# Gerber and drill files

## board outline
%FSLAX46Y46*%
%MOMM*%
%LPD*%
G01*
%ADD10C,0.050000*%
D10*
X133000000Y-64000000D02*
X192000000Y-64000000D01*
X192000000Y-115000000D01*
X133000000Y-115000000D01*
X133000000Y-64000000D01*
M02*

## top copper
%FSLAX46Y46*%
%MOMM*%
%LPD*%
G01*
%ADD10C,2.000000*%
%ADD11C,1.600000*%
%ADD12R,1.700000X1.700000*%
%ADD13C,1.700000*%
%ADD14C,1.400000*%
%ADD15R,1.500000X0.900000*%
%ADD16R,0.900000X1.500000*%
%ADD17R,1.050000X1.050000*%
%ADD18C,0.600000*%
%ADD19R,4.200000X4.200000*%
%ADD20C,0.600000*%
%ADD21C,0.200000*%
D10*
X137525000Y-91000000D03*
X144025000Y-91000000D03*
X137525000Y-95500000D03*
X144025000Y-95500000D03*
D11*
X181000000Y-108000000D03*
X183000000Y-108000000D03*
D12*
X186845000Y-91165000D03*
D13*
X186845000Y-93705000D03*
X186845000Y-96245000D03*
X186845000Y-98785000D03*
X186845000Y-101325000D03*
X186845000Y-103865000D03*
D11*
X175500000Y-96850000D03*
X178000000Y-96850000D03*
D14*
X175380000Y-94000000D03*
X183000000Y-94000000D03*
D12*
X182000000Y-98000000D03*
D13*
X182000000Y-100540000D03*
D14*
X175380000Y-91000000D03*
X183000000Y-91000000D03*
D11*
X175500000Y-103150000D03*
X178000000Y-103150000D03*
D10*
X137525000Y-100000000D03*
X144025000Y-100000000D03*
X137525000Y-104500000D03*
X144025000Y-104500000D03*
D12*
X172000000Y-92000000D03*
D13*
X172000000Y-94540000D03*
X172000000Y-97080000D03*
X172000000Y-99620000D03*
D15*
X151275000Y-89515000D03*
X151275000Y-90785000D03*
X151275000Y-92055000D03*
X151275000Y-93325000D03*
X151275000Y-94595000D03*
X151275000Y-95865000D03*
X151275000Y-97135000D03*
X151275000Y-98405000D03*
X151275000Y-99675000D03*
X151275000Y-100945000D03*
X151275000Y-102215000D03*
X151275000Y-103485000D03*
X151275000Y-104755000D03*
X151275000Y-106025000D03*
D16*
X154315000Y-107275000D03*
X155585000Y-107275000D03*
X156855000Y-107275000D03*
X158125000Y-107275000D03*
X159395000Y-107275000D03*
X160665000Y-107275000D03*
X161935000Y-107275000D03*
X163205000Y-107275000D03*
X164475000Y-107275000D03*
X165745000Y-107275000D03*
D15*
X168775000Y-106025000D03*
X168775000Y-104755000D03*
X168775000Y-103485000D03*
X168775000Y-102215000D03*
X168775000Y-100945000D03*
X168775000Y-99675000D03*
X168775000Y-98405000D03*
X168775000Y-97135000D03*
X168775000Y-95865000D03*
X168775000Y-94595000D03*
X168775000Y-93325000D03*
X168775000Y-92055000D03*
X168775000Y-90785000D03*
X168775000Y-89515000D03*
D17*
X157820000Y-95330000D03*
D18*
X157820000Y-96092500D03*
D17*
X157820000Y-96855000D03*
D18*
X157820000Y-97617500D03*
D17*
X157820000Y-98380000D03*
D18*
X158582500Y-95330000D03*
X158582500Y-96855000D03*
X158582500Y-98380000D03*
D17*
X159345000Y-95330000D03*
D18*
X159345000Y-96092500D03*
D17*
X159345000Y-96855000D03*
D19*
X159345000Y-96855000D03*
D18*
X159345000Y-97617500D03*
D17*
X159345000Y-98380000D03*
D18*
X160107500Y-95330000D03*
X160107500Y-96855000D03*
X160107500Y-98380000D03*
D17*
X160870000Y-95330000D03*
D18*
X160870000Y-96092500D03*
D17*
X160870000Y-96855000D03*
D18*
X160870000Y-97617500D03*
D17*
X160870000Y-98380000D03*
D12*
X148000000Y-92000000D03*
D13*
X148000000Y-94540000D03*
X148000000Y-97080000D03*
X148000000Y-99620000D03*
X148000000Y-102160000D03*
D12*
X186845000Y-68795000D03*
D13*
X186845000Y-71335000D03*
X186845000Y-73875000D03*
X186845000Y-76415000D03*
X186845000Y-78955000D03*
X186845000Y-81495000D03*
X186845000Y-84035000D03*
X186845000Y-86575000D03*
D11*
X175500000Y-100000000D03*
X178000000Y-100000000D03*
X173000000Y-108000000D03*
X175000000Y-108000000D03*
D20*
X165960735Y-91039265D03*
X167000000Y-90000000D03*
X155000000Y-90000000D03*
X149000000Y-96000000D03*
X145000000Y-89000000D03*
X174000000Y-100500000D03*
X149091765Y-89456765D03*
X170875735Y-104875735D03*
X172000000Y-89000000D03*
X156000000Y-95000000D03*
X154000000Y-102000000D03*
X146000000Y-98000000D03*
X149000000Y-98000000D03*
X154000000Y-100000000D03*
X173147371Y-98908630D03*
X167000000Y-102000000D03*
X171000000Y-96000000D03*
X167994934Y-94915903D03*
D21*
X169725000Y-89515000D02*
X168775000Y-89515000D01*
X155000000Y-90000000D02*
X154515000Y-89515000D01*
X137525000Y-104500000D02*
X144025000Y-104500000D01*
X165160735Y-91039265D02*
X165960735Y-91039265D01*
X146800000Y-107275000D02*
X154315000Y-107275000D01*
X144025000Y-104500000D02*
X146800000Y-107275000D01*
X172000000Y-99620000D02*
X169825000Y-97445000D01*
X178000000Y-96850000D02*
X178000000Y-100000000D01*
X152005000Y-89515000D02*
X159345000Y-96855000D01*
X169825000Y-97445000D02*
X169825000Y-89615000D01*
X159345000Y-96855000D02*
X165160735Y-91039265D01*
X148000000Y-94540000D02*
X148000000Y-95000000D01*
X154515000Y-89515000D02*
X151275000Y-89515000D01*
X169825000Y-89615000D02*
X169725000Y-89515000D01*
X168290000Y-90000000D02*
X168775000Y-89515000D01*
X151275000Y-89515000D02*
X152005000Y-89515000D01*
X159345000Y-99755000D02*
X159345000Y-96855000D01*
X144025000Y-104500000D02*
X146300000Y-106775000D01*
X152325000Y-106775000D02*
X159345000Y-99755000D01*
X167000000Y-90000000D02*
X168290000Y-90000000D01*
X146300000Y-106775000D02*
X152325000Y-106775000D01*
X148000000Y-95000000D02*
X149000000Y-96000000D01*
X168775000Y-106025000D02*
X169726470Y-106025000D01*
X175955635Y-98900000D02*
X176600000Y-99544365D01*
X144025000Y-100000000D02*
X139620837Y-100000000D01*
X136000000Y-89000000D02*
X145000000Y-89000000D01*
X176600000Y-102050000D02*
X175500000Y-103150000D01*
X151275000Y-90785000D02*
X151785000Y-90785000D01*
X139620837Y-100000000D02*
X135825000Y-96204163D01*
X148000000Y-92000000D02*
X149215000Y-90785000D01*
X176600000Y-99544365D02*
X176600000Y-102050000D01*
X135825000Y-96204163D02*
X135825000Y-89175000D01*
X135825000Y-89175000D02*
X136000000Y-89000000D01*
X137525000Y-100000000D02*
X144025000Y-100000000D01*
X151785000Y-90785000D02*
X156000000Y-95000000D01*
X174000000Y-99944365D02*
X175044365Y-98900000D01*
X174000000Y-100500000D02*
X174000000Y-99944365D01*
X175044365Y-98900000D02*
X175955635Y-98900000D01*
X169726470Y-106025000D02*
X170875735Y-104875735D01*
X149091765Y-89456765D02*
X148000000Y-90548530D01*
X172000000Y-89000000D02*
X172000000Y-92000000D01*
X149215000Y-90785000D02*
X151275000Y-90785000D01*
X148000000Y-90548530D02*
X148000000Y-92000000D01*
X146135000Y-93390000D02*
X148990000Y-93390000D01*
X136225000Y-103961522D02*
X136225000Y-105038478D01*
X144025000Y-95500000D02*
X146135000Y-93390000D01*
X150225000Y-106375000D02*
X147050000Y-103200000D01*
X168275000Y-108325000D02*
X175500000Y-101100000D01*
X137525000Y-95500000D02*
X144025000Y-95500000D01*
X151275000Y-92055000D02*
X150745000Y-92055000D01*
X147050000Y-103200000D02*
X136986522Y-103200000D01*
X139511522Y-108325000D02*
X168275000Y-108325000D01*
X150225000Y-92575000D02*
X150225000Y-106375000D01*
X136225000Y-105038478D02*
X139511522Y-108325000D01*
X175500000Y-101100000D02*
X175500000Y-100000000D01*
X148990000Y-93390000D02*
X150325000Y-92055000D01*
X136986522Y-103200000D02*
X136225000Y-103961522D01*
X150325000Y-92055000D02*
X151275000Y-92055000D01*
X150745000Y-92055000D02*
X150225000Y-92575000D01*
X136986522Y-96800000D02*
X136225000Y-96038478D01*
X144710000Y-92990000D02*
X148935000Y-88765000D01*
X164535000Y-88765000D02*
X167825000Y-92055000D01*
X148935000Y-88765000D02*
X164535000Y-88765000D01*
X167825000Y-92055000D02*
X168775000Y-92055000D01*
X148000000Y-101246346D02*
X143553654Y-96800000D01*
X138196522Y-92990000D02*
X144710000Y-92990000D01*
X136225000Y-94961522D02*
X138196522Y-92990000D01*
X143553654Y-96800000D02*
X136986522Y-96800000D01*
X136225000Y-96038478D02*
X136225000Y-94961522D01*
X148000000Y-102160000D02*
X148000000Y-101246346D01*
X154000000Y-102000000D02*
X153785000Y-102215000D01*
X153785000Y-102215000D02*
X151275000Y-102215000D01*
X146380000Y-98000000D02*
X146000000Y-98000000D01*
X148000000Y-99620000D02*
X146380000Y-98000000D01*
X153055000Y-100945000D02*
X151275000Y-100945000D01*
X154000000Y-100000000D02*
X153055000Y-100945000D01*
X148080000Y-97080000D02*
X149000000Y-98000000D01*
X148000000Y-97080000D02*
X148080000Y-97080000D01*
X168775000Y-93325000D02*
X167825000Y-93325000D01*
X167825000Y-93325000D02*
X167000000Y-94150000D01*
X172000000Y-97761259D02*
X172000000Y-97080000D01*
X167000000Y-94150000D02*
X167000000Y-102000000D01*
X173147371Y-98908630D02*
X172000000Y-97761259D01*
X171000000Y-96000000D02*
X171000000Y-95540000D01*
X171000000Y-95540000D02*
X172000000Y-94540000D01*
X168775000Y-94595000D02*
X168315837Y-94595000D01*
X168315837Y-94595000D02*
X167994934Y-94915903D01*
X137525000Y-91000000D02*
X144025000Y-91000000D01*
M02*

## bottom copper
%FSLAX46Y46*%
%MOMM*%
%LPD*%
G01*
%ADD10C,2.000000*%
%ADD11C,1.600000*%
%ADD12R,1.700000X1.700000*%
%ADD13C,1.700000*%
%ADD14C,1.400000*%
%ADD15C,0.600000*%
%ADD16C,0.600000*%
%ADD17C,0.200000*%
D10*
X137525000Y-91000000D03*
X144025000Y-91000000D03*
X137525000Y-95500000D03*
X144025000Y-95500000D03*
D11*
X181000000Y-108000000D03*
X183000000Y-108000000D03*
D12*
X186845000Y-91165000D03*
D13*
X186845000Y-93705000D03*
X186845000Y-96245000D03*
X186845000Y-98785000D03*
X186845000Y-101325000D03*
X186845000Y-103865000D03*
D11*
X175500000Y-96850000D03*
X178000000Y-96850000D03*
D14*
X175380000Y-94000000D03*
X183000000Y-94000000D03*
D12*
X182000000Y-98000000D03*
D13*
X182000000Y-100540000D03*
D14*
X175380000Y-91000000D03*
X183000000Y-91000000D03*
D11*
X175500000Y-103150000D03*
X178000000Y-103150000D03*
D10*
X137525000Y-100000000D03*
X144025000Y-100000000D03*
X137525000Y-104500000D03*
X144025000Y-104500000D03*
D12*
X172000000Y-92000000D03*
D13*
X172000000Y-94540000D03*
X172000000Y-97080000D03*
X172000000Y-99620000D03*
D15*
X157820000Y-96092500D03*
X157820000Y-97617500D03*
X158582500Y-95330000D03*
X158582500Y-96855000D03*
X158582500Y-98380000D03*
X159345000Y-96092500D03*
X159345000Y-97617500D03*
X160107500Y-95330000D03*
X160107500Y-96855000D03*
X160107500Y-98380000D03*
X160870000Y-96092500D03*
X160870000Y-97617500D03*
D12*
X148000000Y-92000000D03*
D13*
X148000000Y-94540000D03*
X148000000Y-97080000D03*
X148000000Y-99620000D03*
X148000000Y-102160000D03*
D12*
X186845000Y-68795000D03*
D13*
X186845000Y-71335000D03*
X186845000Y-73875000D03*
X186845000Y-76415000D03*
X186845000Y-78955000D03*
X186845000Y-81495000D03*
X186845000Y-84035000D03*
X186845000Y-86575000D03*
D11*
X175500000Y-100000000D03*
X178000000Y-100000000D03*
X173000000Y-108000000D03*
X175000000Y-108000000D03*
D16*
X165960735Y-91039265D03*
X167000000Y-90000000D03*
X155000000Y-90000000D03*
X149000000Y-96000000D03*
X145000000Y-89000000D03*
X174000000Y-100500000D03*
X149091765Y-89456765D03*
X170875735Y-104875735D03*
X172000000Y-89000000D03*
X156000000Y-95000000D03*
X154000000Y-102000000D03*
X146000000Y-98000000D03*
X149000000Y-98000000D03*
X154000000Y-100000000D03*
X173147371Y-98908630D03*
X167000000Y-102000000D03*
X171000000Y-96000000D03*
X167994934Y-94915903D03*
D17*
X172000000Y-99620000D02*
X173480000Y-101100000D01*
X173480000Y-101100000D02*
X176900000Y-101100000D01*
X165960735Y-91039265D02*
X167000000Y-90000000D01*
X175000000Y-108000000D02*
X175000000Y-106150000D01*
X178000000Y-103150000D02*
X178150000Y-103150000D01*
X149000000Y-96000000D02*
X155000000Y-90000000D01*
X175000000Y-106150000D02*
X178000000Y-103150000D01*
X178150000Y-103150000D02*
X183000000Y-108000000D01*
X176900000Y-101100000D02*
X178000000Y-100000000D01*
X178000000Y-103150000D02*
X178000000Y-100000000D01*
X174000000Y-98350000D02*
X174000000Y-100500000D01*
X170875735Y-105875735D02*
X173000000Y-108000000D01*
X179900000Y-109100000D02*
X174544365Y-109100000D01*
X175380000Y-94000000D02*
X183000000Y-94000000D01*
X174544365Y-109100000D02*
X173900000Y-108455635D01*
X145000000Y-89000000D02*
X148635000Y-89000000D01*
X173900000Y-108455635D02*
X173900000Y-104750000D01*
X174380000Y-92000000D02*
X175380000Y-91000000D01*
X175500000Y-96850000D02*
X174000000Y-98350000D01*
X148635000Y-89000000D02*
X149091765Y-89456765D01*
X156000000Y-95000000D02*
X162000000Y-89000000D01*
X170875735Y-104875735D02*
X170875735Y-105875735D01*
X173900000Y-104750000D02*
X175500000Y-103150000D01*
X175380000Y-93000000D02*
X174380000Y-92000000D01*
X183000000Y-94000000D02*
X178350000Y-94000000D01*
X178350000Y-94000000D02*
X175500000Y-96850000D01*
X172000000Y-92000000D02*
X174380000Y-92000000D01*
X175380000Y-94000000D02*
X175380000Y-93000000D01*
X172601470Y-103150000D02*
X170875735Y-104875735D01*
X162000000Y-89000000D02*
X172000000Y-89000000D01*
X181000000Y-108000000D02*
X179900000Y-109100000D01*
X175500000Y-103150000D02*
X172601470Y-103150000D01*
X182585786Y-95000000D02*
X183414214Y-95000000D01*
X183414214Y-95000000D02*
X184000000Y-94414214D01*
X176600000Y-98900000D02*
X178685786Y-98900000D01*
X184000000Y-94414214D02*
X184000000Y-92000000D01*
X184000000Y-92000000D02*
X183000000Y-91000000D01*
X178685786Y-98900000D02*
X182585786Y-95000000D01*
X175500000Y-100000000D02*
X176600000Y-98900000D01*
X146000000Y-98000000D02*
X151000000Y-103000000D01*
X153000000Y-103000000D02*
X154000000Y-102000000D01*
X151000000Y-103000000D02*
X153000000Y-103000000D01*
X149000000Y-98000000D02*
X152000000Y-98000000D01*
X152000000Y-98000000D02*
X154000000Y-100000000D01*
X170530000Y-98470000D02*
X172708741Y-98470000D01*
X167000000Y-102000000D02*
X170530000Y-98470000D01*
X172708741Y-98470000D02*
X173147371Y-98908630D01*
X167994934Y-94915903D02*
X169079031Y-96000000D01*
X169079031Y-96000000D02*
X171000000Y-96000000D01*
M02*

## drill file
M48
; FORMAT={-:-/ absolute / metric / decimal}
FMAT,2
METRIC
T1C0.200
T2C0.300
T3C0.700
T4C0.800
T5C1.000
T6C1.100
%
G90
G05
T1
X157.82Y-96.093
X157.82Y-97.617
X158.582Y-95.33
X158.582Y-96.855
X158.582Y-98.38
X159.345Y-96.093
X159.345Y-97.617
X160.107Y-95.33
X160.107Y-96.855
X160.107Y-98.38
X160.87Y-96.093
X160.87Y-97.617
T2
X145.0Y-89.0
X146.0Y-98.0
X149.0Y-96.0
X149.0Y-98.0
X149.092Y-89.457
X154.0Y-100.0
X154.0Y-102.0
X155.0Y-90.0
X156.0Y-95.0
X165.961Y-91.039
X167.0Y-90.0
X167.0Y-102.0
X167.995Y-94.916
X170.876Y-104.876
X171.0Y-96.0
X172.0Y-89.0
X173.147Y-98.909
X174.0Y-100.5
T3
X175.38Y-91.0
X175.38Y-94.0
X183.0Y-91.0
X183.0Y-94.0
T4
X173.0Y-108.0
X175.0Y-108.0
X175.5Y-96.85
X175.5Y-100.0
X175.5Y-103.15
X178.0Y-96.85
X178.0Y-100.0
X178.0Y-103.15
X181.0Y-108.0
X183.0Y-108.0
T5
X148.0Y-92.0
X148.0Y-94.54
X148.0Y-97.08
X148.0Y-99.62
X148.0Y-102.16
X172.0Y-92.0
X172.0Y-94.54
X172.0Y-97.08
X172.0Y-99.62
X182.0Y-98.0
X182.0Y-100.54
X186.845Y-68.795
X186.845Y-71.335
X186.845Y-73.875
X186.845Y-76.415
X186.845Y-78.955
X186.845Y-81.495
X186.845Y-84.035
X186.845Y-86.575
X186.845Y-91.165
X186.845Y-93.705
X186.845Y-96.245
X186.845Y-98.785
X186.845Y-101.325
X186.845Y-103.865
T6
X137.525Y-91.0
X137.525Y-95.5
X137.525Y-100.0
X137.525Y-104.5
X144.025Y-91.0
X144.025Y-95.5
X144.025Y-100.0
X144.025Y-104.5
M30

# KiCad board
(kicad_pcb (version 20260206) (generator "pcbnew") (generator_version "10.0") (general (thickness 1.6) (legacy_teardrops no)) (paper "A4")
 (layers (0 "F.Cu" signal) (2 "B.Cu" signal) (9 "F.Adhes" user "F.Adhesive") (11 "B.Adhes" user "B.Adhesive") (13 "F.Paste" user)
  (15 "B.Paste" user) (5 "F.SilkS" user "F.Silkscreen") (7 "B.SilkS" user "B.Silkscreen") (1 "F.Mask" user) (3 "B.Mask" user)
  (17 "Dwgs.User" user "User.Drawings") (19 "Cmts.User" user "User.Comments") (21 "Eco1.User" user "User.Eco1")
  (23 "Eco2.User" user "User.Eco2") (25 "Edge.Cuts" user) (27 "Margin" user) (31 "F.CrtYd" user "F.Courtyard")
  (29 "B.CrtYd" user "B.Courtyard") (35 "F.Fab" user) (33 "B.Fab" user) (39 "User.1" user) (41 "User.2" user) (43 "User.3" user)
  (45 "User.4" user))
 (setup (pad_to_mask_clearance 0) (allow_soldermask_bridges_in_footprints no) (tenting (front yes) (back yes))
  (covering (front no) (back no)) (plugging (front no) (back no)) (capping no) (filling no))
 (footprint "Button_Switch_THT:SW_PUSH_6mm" (layer "F.Cu") (at 137.525 91)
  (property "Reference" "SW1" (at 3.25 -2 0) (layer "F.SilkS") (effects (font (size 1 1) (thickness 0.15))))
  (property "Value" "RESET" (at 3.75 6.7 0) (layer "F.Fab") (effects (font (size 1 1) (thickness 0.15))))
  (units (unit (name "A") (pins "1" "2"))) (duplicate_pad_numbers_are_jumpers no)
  (pad "1" thru_hole circle (at 0 0 90) (size 2 2) (drill 1.1) (layers "*.Cu" "*.Mask") (remove_unused_layers no)
   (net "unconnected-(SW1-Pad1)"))
  (pad "1" thru_hole circle (at 6.5 0 90) (size 2 2) (drill 1.1) (layers "*.Cu" "*.Mask") (remove_unused_layers no)
   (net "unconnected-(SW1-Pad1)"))
  (pad "2" thru_hole circle (at 0 4.5 90) (size 2 2) (drill 1.1) (layers "*.Cu" "*.Mask") (remove_unused_layers no) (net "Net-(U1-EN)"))
  (pad "2" thru_hole circle (at 6.5 4.5 90) (size 2 2) (drill 1.1) (layers "*.Cu" "*.Mask") (remove_unused_layers no) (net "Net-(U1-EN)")))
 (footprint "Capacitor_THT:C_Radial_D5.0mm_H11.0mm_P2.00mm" (layer "F.Cu") (at 181 108)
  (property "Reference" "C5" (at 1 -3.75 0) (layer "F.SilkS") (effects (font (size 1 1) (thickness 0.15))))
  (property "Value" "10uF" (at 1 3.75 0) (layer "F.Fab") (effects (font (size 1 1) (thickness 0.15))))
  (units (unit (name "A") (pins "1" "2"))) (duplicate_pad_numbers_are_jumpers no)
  (pad "1" thru_hole circle (at 0 0) (size 1.6 1.6) (drill 0.8) (layers "*.Cu" "*.Mask") (remove_unused_layers no) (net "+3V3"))
  (pad "2" thru_hole circle (at 2 0) (size 1.6 1.6) (drill 0.8) (layers "*.Cu" "*.Mask") (remove_unused_layers no) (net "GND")))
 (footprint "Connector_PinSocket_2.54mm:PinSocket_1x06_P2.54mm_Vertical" (layer "F.Cu") (at 186.845 91.165)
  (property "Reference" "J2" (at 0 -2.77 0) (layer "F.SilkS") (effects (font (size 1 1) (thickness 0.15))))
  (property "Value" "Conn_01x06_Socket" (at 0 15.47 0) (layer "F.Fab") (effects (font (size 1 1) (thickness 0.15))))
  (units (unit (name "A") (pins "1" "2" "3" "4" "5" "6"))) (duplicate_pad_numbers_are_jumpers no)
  (pad "1" thru_hole rect (at 0 0) (size 1.7 1.7) (drill 1) (layers "*.Cu" "*.Mask") (remove_unused_layers no)
   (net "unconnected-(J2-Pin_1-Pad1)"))
  (pad "2" thru_hole circle (at 0 2.54) (size 1.7 1.7) (drill 1) (layers "*.Cu" "*.Mask") (remove_unused_layers no)
   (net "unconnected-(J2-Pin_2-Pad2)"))
  (pad "3" thru_hole circle (at 0 5.08) (size 1.7 1.7) (drill 1) (layers "*.Cu" "*.Mask") (remove_unused_layers no)
   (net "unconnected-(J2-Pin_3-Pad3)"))
  (pad "4" thru_hole circle (at 0 7.62) (size 1.7 1.7) (drill 1) (layers "*.Cu" "*.Mask") (remove_unused_layers no)
   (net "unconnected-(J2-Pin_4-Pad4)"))
  (pad "5" thru_hole circle (at 0 10.16) (size 1.7 1.7) (drill 1) (layers "*.Cu" "*.Mask") (remove_unused_layers no)
   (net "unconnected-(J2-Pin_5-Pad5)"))
  (pad "6" thru_hole circle (at 0 12.7) (size 1.7 1.7) (drill 1) (layers "*.Cu" "*.Mask") (remove_unused_layers no)
   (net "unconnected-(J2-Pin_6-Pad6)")))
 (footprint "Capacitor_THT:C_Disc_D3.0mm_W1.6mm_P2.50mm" (layer "F.Cu") (at 175.5 96.85)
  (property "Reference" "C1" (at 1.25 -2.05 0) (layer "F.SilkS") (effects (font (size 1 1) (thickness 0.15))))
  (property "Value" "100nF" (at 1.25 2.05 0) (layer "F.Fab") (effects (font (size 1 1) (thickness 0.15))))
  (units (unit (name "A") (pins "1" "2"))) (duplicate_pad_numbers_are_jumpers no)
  (pad "1" thru_hole circle (at 0 0) (size 1.6 1.6) (drill 0.8) (layers "*.Cu" "*.Mask") (remove_unused_layers no) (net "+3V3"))
  (pad "2" thru_hole circle (at 2.5 0) (size 1.6 1.6) (drill 0.8) (layers "*.Cu" "*.Mask") (remove_unused_layers no) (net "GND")))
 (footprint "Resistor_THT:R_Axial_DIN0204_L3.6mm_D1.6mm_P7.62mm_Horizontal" (layer "F.Cu") (at 175.38 94)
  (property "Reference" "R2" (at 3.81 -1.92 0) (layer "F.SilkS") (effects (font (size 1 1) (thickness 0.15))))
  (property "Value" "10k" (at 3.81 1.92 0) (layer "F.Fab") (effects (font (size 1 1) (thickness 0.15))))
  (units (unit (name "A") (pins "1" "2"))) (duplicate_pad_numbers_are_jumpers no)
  (pad "1" thru_hole circle (at 0 0) (size 1.4 1.4) (drill 0.7) (layers "*.Cu" "*.Mask") (remove_unused_layers no) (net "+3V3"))
  (pad "2" thru_hole circle (at 7.62 0) (size 1.4 1.4) (drill 0.7) (layers "*.Cu" "*.Mask") (remove_unused_layers no) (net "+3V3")))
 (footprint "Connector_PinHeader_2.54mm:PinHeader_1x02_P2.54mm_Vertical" (layer "F.Cu") (at 182 98)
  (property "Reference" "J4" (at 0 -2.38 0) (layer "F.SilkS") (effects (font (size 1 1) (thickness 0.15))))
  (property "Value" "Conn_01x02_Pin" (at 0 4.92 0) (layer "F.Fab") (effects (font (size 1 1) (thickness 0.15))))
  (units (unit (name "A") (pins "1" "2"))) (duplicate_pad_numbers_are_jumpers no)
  (pad "1" thru_hole rect (at 0 0) (size 1.7 1.7) (drill 1) (layers "*.Cu" "*.Mask") (remove_unused_layers no) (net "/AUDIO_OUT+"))
  (pad "2" thru_hole circle (at 0 2.54) (size 1.7 1.7) (drill 1) (layers "*.Cu" "*.Mask") (remove_unused_layers no) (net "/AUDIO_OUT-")))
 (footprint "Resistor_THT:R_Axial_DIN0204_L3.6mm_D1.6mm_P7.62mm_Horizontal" (layer "F.Cu") (at 175.38 91)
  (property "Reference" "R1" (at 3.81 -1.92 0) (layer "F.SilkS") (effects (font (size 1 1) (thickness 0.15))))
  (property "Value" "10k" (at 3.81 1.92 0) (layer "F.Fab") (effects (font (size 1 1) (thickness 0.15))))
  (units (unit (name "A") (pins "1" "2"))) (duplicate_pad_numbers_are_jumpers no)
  (pad "1" thru_hole circle (at 0 0) (size 1.4 1.4) (drill 0.7) (layers "*.Cu" "*.Mask") (remove_unused_layers no) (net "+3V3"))
  (pad "2" thru_hole circle (at 7.62 0) (size 1.4 1.4) (drill 0.7) (layers "*.Cu" "*.Mask") (remove_unused_layers no) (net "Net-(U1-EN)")))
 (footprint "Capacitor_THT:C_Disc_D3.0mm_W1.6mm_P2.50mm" (layer "F.Cu") (at 175.5 103.15)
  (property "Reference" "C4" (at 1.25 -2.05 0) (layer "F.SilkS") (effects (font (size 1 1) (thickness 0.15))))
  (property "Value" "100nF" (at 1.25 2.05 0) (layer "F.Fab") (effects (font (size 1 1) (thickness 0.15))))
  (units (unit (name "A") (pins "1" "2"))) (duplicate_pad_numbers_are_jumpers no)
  (pad "1" thru_hole circle (at 0 0) (size 1.6 1.6) (drill 0.8) (layers "*.Cu" "*.Mask") (remove_unused_layers no) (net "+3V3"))
  (pad "2" thru_hole circle (at 2.5 0) (size 1.6 1.6) (drill 0.8) (layers "*.Cu" "*.Mask") (remove_unused_layers no) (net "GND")))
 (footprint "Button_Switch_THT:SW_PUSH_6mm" (layer "F.Cu") (at 137.525 100)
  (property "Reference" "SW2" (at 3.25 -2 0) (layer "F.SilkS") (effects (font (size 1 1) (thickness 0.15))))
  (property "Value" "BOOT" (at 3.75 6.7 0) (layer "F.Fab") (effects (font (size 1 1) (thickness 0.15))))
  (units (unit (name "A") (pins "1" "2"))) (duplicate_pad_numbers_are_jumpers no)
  (pad "1" thru_hole circle (at 0 0 90) (size 2 2) (drill 1.1) (layers "*.Cu" "*.Mask") (remove_unused_layers no) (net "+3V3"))
  (pad "1" thru_hole circle (at 6.5 0 90) (size 2 2) (drill 1.1) (layers "*.Cu" "*.Mask") (remove_unused_layers no) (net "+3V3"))
  (pad "2" thru_hole circle (at 0 4.5 90) (size 2 2) (drill 1.1) (layers "*.Cu" "*.Mask") (remove_unused_layers no) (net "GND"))
  (pad "2" thru_hole circle (at 6.5 4.5 90) (size 2 2) (drill 1.1) (layers "*.Cu" "*.Mask") (remove_unused_layers no) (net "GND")))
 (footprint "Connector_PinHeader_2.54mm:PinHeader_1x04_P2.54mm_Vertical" (layer "F.Cu") (at 172 92)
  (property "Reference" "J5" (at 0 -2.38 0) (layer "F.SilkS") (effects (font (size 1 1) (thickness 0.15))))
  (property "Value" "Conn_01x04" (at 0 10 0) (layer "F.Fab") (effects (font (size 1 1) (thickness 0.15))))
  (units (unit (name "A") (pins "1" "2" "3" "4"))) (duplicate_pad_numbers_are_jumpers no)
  (pad "1" thru_hole rect (at 0 0) (size 1.7 1.7) (drill 1) (layers "*.Cu" "*.Mask") (remove_unused_layers no) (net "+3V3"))
  (pad "2" thru_hole circle (at 0 2.54) (size 1.7 1.7) (drill 1) (layers "*.Cu" "*.Mask") (remove_unused_layers no) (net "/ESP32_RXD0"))
  (pad "3" thru_hole circle (at 0 5.08) (size 1.7 1.7) (drill 1) (layers "*.Cu" "*.Mask") (remove_unused_layers no) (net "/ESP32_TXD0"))
  (pad "4" thru_hole circle (at 0 7.62) (size 1.7 1.7) (drill 1) (layers "*.Cu" "*.Mask") (remove_unused_layers no) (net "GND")))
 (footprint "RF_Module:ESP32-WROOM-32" (layer "F.Cu") (at 160.025 97.765)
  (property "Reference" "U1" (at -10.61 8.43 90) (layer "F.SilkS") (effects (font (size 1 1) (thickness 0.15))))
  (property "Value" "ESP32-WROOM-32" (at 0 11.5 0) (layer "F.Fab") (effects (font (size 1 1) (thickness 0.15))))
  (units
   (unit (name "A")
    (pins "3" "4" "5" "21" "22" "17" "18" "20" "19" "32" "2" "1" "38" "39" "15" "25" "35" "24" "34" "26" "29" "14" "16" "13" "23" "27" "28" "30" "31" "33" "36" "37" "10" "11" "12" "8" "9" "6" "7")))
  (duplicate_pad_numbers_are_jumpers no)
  (pad "1" smd rect (at -8.75 -8.25) (size 1.5 0.9) (layers "F.Cu" "F.Mask" "F.Paste") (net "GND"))
  (pad "2" smd rect (at -8.75 -6.98) (size 1.5 0.9) (layers "F.Cu" "F.Mask" "F.Paste") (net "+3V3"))
  (pad "3" smd rect (at -8.75 -5.71) (size 1.5 0.9) (layers "F.Cu" "F.Mask" "F.Paste") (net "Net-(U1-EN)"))
  (pad "4" smd rect (at -8.75 -4.44) (size 1.5 0.9) (layers "F.Cu" "F.Mask" "F.Paste") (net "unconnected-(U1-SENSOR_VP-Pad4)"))
  (pad "5" smd rect (at -8.75 -3.17) (size 1.5 0.9) (layers "F.Cu" "F.Mask" "F.Paste") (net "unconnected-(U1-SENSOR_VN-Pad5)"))
  (pad "6" smd rect (at -8.75 -1.9) (size 1.5 0.9) (layers "F.Cu" "F.Mask" "F.Paste") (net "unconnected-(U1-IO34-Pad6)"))
  (pad "7" smd rect (at -8.75 -0.63) (size 1.5 0.9) (layers "F.Cu" "F.Mask" "F.Paste") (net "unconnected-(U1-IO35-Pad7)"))
  (pad "8" smd rect (at -8.75 0.64) (size 1.5 0.9) (layers "F.Cu" "F.Mask" "F.Paste") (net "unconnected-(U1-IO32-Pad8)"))
  (pad "9" smd rect (at -8.75 1.91) (size 1.5 0.9) (layers "F.Cu" "F.Mask" "F.Paste") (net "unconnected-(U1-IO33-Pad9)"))
  (pad "10" smd rect (at -8.75 3.18) (size 1.5 0.9) (layers "F.Cu" "F.Mask" "F.Paste") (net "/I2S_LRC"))
  (pad "11" smd rect (at -8.75 4.45) (size 1.5 0.9) (layers "F.Cu" "F.Mask" "F.Paste") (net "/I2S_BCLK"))
  (pad "12" smd rect (at -8.75 5.72) (size 1.5 0.9) (layers "F.Cu" "F.Mask" "F.Paste") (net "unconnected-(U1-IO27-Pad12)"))
  (pad "13" smd rect (at -8.75 6.99) (size 1.5 0.9) (layers "F.Cu" "F.Mask" "F.Paste") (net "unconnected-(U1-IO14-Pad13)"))
  (pad "14" smd rect (at -8.75 8.26) (size 1.5 0.9) (layers "F.Cu" "F.Mask" "F.Paste") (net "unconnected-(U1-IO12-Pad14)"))
  (pad "15" smd rect (at -5.71 9.51 90) (size 1.5 0.9) (layers "F.Cu" "F.Mask" "F.Paste") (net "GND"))
  (pad "16" smd rect (at -4.44 9.51 90) (size 1.5 0.9) (layers "F.Cu" "F.Mask" "F.Paste") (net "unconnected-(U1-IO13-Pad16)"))
  (pad "17" smd rect (at -3.17 9.51 90) (size 1.5 0.9) (layers "F.Cu" "F.Mask" "F.Paste") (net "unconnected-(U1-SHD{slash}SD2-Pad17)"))
  (pad "18" smd rect (at -1.9 9.51 90) (size 1.5 0.9) (layers "F.Cu" "F.Mask" "F.Paste") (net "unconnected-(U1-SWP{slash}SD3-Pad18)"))
  (pad "19" smd rect (at -0.63 9.51 90) (size 1.5 0.9) (layers "F.Cu" "F.Mask" "F.Paste") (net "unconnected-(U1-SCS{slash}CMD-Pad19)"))
  (pad "20" smd rect (at 0.64 9.51 90) (size 1.5 0.9) (layers "F.Cu" "F.Mask" "F.Paste") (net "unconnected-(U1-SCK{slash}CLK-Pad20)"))
  (pad "21" smd rect (at 1.91 9.51 90) (size 1.5 0.9) (layers "F.Cu" "F.Mask" "F.Paste") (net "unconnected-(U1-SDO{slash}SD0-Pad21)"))
  (pad "22" smd rect (at 3.18 9.51 90) (size 1.5 0.9) (layers "F.Cu" "F.Mask" "F.Paste") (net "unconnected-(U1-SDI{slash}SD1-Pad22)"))
  (pad "23" smd rect (at 4.45 9.51 90) (size 1.5 0.9) (layers "F.Cu" "F.Mask" "F.Paste") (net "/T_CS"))
  (pad "24" smd rect (at 5.72 9.51 90) (size 1.5 0.9) (layers "F.Cu" "F.Mask" "F.Paste") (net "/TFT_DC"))
  (pad "25" smd rect (at 8.75 8.26) (size 1.5 0.9) (layers "F.Cu" "F.Mask" "F.Paste") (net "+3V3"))
  (pad "26" smd rect (at 8.75 6.99) (size 1.5 0.9) (layers "F.Cu" "F.Mask" "F.Paste") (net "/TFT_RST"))
  (pad "27" smd rect (at 8.75 5.72) (size 1.5 0.9) (layers "F.Cu" "F.Mask" "F.Paste") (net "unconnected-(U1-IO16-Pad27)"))
  (pad "28" smd rect (at 8.75 4.45) (size 1.5 0.9) (layers "F.Cu" "F.Mask" "F.Paste") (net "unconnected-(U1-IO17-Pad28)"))
  (pad "29" smd rect (at 8.75 3.18) (size 1.5 0.9) (layers "F.Cu" "F.Mask" "F.Paste") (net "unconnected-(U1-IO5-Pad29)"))
  (pad "30" smd rect (at 8.75 1.91) (size 1.5 0.9) (layers "F.Cu" "F.Mask" "F.Paste") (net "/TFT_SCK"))
  (pad "31" smd rect (at 8.75 0.64) (size 1.5 0.9) (layers "F.Cu" "F.Mask" "F.Paste") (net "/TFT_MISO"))
  (pad "32" smd rect (at 8.75 -0.63) (size 1.5 0.9) (layers "F.Cu" "F.Mask" "F.Paste") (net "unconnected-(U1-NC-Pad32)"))
  (pad "33" smd rect (at 8.75 -1.9) (size 1.5 0.9) (layers "F.Cu" "F.Mask" "F.Paste") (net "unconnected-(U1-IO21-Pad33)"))
  (pad "34" smd rect (at 8.75 -3.17) (size 1.5 0.9) (layers "F.Cu" "F.Mask" "F.Paste") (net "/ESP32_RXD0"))
  (pad "35" smd rect (at 8.75 -4.44) (size 1.5 0.9) (layers "F.Cu" "F.Mask" "F.Paste") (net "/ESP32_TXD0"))
  (pad "36" smd rect (at 8.75 -5.71) (size 1.5 0.9) (layers "F.Cu" "F.Mask" "F.Paste") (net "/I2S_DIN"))
  (pad "37" smd rect (at 8.75 -6.98) (size 1.5 0.9) (layers "F.Cu" "F.Mask" "F.Paste") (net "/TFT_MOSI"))
  (pad "38" smd rect (at 8.75 -8.25) (size 1.5 0.9) (layers "F.Cu" "F.Mask" "F.Paste") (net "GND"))
  (pad "39" smd rect (at -2.205 -2.435) (size 1.05 1.05) (layers "F.Cu" "F.Paste") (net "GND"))
  (pad "39" thru_hole circle (at -2.205 -1.6725) (size 0.6 0.6) (drill 0.2) (layers "*.Cu" "F.Mask") (remove_unused_layers no) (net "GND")
   (zone_connect 2))
  (pad "39" smd rect (at -2.205 -0.91) (size 1.05 1.05) (layers "F.Cu" "F.Paste") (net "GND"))
  (pad "39" thru_hole circle (at -2.205 -0.1475) (size 0.6 0.6) (drill 0.2) (layers "*.Cu" "F.Mask") (remove_unused_layers no) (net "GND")
   (zone_connect 2))
  (pad "39" smd rect (at -2.205 0.615) (size 1.05 1.05) (layers "F.Cu" "F.Paste") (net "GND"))
  (pad "39" thru_hole circle (at -1.4425 -2.435) (size 0.6 0.6) (drill 0.2) (layers "*.Cu" "F.Mask") (remove_unused_layers no) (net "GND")
   (zone_connect 2))
  (pad "39" thru_hole circle (at -1.4425 -0.91) (size 0.6 0.6) (drill 0.2) (layers "*.Cu" "F.Mask") (remove_unused_layers no) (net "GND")
   (zone_connect 2))
  (pad "39" thru_hole circle (at -1.4425 0.615) (size 0.6 0.6) (drill 0.2) (layers "*.Cu" "F.Mask") (remove_unused_layers no) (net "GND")
   (zone_connect 2))
  (pad "39" smd rect (at -0.68 -2.435) (size 1.05 1.05) (layers "F.Cu" "F.Paste") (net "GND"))
  (pad "39" thru_hole circle (at -0.68 -1.6725) (size 0.6 0.6) (drill 0.2) (layers "*.Cu" "F.Mask") (remove_unused_layers no) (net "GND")
   (zone_connect 2))
  (pad "39" smd rect (at -0.68 -0.91) (size 1.05 1.05) (layers "F.Cu" "F.Paste") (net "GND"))
  (pad "39" smd rect (at -0.68 -0.91) (size 4.2 4.2) (layers "F.Cu" "F.Mask") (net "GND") (zone_connect 2))
  (pad "39" thru_hole circle (at -0.68 -0.1475) (size 0.6 0.6) (drill 0.2) (layers "*.Cu" "F.Mask") (remove_unused_layers no) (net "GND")
   (zone_connect 2))
  (pad "39" smd rect (at -0.68 0.615) (size 1.05 1.05) (layers "F.Cu" "F.Paste") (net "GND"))
  (pad "39" thru_hole circle (at 0.0825 -2.435) (size 0.6 0.6) (drill 0.2) (layers "*.Cu" "F.Mask") (remove_unused_layers no) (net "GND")
   (zone_connect 2))
  (pad "39" thru_hole circle (at 0.0825 -0.91) (size 0.6 0.6) (drill 0.2) (layers "*.Cu" "F.Mask") (remove_unused_layers no) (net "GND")
   (zone_connect 2))
  (pad "39" thru_hole circle (at 0.0825 0.615) (size 0.6 0.6) (drill 0.2) (layers "*.Cu" "F.Mask") (remove_unused_layers no) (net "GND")
   (zone_connect 2))
  (pad "39" smd rect (at 0.845 -2.435) (size 1.05 1.05) (layers "F.Cu" "F.Paste") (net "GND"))
  (pad "39" thru_hole circle (at 0.845 -1.6725) (size 0.6 0.6) (drill 0.2) (layers "*.Cu" "F.Mask") (remove_unused_layers no) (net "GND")
   (zone_connect 2))
  (pad "39" smd rect (at 0.845 -0.91) (size 1.05 1.05) (layers "F.Cu" "F.Paste") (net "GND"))
  (pad "39" thru_hole circle (at 0.845 -0.1475) (size 0.6 0.6) (drill 0.2) (layers "*.Cu" "F.Mask") (remove_unused_layers no) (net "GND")
   (zone_connect 2))
  (pad "39" smd rect (at 0.845 0.615) (size 1.05 1.05) (layers "F.Cu" "F.Paste") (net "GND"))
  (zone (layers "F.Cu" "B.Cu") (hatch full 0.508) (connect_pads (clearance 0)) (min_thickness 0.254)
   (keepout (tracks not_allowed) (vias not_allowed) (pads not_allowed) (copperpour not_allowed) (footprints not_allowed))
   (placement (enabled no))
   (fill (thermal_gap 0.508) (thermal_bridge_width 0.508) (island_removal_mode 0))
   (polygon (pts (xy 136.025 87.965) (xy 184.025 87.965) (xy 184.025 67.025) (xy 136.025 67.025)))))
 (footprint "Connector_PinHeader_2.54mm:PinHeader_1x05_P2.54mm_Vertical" (layer "F.Cu") (at 148 92)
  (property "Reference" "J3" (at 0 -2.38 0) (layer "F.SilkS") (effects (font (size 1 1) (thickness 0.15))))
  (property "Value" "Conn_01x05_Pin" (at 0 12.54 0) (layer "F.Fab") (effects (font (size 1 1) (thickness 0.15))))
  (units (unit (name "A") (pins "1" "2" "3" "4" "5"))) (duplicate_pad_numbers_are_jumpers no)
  (pad "1" thru_hole rect (at 0 0) (size 1.7 1.7) (drill 1) (layers "*.Cu" "*.Mask") (remove_unused_layers no) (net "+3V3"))
  (pad "2" thru_hole circle (at 0 2.54) (size 1.7 1.7) (drill 1) (layers "*.Cu" "*.Mask") (remove_unused_layers no) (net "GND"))
  (pad "3" thru_hole circle (at 0 5.08) (size 1.7 1.7) (drill 1) (layers "*.Cu" "*.Mask") (remove_unused_layers no) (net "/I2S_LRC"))
  (pad "4" thru_hole circle (at 0 7.62) (size 1.7 1.7) (drill 1) (layers "*.Cu" "*.Mask") (remove_unused_layers no) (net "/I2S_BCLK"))
  (pad "5" thru_hole circle (at 0 10.16) (size 1.7 1.7) (drill 1) (layers "*.Cu" "*.Mask") (remove_unused_layers no) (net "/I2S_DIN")))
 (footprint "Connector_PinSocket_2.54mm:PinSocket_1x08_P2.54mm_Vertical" (layer "F.Cu") (at 186.845 68.795)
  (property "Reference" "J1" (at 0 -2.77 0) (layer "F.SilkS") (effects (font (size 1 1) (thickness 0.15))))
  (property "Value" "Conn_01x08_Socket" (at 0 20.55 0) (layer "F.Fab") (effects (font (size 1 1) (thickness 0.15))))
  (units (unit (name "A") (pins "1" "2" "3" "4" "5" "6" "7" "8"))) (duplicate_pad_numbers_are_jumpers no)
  (pad "1" thru_hole rect (at 0 0) (size 1.7 1.7) (drill 1) (layers "*.Cu" "*.Mask") (remove_unused_layers no)
   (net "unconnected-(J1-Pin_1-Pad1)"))
  (pad "2" thru_hole circle (at 0 2.54) (size 1.7 1.7) (drill 1) (layers "*.Cu" "*.Mask") (remove_unused_layers no)
   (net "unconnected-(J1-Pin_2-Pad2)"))
  (pad "3" thru_hole circle (at 0 5.08) (size 1.7 1.7) (drill 1) (layers "*.Cu" "*.Mask") (remove_unused_layers no)
   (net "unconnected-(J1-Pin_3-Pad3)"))
  (pad "4" thru_hole circle (at 0 7.62) (size 1.7 1.7) (drill 1) (layers "*.Cu" "*.Mask") (remove_unused_layers no)
   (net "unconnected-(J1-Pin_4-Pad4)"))
  (pad "5" thru_hole circle (at 0 10.16) (size 1.7 1.7) (drill 1) (layers "*.Cu" "*.Mask") (remove_unused_layers no)
   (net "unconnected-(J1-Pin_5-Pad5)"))
  (pad "6" thru_hole circle (at 0 12.7) (size 1.7 1.7) (drill 1) (layers "*.Cu" "*.Mask") (remove_unused_layers no)
   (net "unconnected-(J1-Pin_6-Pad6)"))
  (pad "7" thru_hole circle (at 0 15.24) (size 1.7 1.7) (drill 1) (layers "*.Cu" "*.Mask") (remove_unused_layers no)
   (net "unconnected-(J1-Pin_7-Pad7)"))
  (pad "8" thru_hole circle (at 0 17.78) (size 1.7 1.7) (drill 1) (layers "*.Cu" "*.Mask") (remove_unused_layers no)
   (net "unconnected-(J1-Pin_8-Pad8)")))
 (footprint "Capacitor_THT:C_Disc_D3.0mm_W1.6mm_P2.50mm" (layer "F.Cu") (at 175.5 100)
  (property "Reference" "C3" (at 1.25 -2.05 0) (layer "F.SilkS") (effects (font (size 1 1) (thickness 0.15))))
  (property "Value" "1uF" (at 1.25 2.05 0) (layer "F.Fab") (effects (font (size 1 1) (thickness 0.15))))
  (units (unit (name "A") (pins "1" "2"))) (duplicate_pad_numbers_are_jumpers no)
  (pad "1" thru_hole circle (at 0 0) (size 1.6 1.6) (drill 0.8) (layers "*.Cu" "*.Mask") (remove_unused_layers no) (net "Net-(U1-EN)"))
  (pad "2" thru_hole circle (at 2.5 0) (size 1.6 1.6) (drill 0.8) (layers "*.Cu" "*.Mask") (remove_unused_layers no) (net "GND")))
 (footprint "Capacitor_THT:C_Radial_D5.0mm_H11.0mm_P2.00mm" (layer "F.Cu") (at 173 108)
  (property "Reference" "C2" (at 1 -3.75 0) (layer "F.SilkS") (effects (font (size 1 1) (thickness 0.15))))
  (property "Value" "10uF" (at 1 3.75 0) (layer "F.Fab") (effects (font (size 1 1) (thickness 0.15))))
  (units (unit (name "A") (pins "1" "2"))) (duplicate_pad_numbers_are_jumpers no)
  (pad "1" thru_hole circle (at 0 0) (size 1.6 1.6) (drill 0.8) (layers "*.Cu" "*.Mask") (remove_unused_layers no) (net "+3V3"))
  (pad "2" thru_hole circle (at 2 0) (size 1.6 1.6) (drill 0.8) (layers "*.Cu" "*.Mask") (remove_unused_layers no) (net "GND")))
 (gr_rect (start 133 64) (end 192 115) (stroke (width 0.05) (type default)) (fill no) (layer "Edge.Cuts"))
 (segment (start 169.725 89.515) (end 168.775 89.515) (width 0.2) (layer "F.Cu") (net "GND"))
 (segment (start 155 90) (end 154.515 89.515) (width 0.2) (layer "F.Cu") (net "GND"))
 (segment (start 137.525 104.5) (end 144.025 104.5) (width 0.2) (layer "F.Cu") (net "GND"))
 (segment (start 165.160735 91.039265) (end 165.960735 91.039265) (width 0.2) (layer "F.Cu") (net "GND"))
 (segment (start 146.8 107.275) (end 154.315 107.275) (width 0.2) (layer "F.Cu") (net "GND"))
 (segment (start 144.025 104.5) (end 146.8 107.275) (width 0.2) (layer "F.Cu") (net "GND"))
 (segment (start 172 99.62) (end 169.825 97.445) (width 0.2) (layer "F.Cu") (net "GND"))
 (segment (start 178 96.85) (end 178 100) (width 0.2) (layer "F.Cu") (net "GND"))
 (segment (start 152.005 89.515) (end 159.345 96.855) (width 0.2) (layer "F.Cu") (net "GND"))
 (segment (start 169.825 97.445) (end 169.825 89.615) (width 0.2) (layer "F.Cu") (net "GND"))
 (segment (start 159.345 96.855) (end 165.160735 91.039265) (width 0.2) (layer "F.Cu") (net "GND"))
 (segment (start 148 94.54) (end 148 95) (width 0.2) (layer "F.Cu") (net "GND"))
 (segment (start 154.515 89.515) (end 151.275 89.515) (width 0.2) (layer "F.Cu") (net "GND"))
 (segment (start 169.825 89.615) (end 169.725 89.515) (width 0.2) (layer "F.Cu") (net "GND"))
 (segment (start 168.29 90) (end 168.775 89.515) (width 0.2) (layer "F.Cu") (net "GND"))
 (segment (start 151.275 89.515) (end 152.005 89.515) (width 0.2) (layer "F.Cu") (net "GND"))
 (segment (start 159.345 99.755) (end 159.345 96.855) (width 0.2) (layer "F.Cu") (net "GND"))
 (segment (start 144.025 104.5) (end 146.3 106.775) (width 0.2) (layer "F.Cu") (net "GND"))
 (segment (start 152.325 106.775) (end 159.345 99.755) (width 0.2) (layer "F.Cu") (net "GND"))
 (segment (start 167 90) (end 168.29 90) (width 0.2) (layer "F.Cu") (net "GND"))
 (segment (start 146.3 106.775) (end 152.325 106.775) (width 0.2) (layer "F.Cu") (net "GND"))
 (segment (start 148 95) (end 149 96) (width 0.2) (layer "F.Cu") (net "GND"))
 (via (at 165.960735 91.039265) (size 0.6) (drill 0.3) (layers "F.Cu" "B.Cu") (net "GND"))
 (via (at 167 90) (size 0.6) (drill 0.3) (layers "F.Cu" "B.Cu") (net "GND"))
 (via (at 155 90) (size 0.6) (drill 0.3) (layers "F.Cu" "B.Cu") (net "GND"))
 (via (at 149 96) (size 0.6) (drill 0.3) (layers "F.Cu" "B.Cu") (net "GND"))
 (segment (start 172 99.62) (end 173.48 101.1) (width 0.2) (layer "B.Cu") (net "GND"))
 (segment (start 173.48 101.1) (end 176.9 101.1) (width 0.2) (layer "B.Cu") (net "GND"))
 (segment (start 165.960735 91.039265) (end 167 90) (width 0.2) (layer "B.Cu") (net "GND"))
 (segment (start 175 108) (end 175 106.15) (width 0.2) (layer "B.Cu") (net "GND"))
 (segment (start 178 103.15) (end 178.15 103.15) (width 0.2) (layer "B.Cu") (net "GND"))
 (segment (start 149 96) (end 155 90) (width 0.2) (layer "B.Cu") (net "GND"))
 (segment (start 175 106.15) (end 178 103.15) (width 0.2) (layer "B.Cu") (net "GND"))
 (segment (start 178.15 103.15) (end 183 108) (width 0.2) (layer "B.Cu") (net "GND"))
 (segment (start 176.9 101.1) (end 178 100) (width 0.2) (layer "B.Cu") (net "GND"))
 (segment (start 178 103.15) (end 178 100) (width 0.2) (layer "B.Cu") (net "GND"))
 (segment (start 168.775 106.025) (end 169.72647 106.025) (width 0.2) (layer "F.Cu") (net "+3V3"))
 (segment (start 175.955635 98.9) (end 176.6 99.544365) (width 0.2) (layer "F.Cu") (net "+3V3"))
 (segment (start 144.025 100) (end 139.620837 100) (width 0.2) (layer "F.Cu") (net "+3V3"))
 (segment (start 136 89) (end 145 89) (width 0.2) (layer "F.Cu") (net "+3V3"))
 (segment (start 176.6 102.05) (end 175.5 103.15) (width 0.2) (layer "F.Cu") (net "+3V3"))
 (segment (start 151.275 90.785) (end 151.785 90.785) (width 0.2) (layer "F.Cu") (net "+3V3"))
 (segment (start 139.620837 100) (end 135.825 96.204163) (width 0.2) (layer "F.Cu") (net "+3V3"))
 (segment (start 148 92) (end 149.215 90.785) (width 0.2) (layer "F.Cu") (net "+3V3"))
 (segment (start 176.6 99.544365) (end 176.6 102.05) (width 0.2) (layer "F.Cu") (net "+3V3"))
 (segment (start 135.825 96.204163) (end 135.825 89.175) (width 0.2) (layer "F.Cu") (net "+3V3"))
 (segment (start 135.825 89.175) (end 136 89) (width 0.2) (layer "F.Cu") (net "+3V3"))
 (segment (start 137.525 100) (end 144.025 100) (width 0.2) (layer "F.Cu") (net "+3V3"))
 (segment (start 151.785 90.785) (end 156 95) (width 0.2) (layer "F.Cu") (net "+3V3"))
 (segment (start 174 99.944365) (end 175.044365 98.9) (width 0.2) (layer "F.Cu") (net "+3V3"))
 (segment (start 174 100.5) (end 174 99.944365) (width 0.2) (layer "F.Cu") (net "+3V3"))
 (segment (start 175.044365 98.9) (end 175.955635 98.9) (width 0.2) (layer "F.Cu") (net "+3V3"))
 (segment (start 169.72647 106.025) (end 170.875735 104.875735) (width 0.2) (layer "F.Cu") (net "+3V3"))
 (segment (start 149.091765 89.456765) (end 148 90.54853) (width 0.2) (layer "F.Cu") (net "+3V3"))
 (segment (start 172 89) (end 172 92) (width 0.2) (layer "F.Cu") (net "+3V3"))
 (segment (start 149.215 90.785) (end 151.275 90.785) (width 0.2) (layer "F.Cu") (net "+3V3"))
 (segment (start 148 90.54853) (end 148 92) (width 0.2) (layer "F.Cu") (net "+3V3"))
 (via (at 145 89) (size 0.6) (drill 0.3) (layers "F.Cu" "B.Cu") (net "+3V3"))
 (via (at 174 100.5) (size 0.6) (drill 0.3) (layers "F.Cu" "B.Cu") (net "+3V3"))
 (via (at 149.091765 89.456765) (size 0.6) (drill 0.3) (layers "F.Cu" "B.Cu") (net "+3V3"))
 (via (at 170.875735 104.875735) (size 0.6) (drill 0.3) (layers "F.Cu" "B.Cu") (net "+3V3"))
 (via (at 172 89) (size 0.6) (drill 0.3) (layers "F.Cu" "B.Cu") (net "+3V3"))
 (via (at 156 95) (size 0.6) (drill 0.3) (layers "F.Cu" "B.Cu") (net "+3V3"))
 (segment (start 174 98.35) (end 174 100.5) (width 0.2) (layer "B.Cu") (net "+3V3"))
 (segment (start 170.875735 105.875735) (end 173 108) (width 0.2) (layer "B.Cu") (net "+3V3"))
 (segment (start 179.9 109.1) (end 174.544365 109.1) (width 0.2) (layer "B.Cu") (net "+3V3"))
 (segment (start 175.38 94) (end 183 94) (width 0.2) (layer "B.Cu") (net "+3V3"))
 (segment (start 174.544365 109.1) (end 173.9 108.455635) (width 0.2) (layer "B.Cu") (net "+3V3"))
 (segment (start 145 89) (end 148.635 89) (width 0.2) (layer "B.Cu") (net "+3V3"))
 (segment (start 173.9 108.455635) (end 173.9 104.75) (width 0.2) (layer "B.Cu") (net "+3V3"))
 (segment (start 174.38 92) (end 175.38 91) (width 0.2) (layer "B.Cu") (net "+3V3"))
 (segment (start 175.5 96.85) (end 174 98.35) (width 0.2) (layer "B.Cu") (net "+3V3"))
 (segment (start 148.635 89) (end 149.091765 89.456765) (width 0.2) (layer "B.Cu") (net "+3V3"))
 (segment (start 156 95) (end 162 89) (width 0.2) (layer "B.Cu") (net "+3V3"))
 (segment (start 170.875735 104.875735) (end 170.875735 105.875735) (width 0.2) (layer "B.Cu") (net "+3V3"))
 (segment (start 173.9 104.75) (end 175.5 103.15) (width 0.2) (layer "B.Cu") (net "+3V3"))
 (segment (start 175.38 93) (end 174.38 92) (width 0.2) (layer "B.Cu") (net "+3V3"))
 (segment (start 183 94) (end 178.35 94) (width 0.2) (layer "B.Cu") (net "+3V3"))
 (segment (start 178.35 94) (end 175.5 96.85) (width 0.2) (layer "B.Cu") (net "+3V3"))
 (segment (start 172 92) (end 174.38 92) (width 0.2) (layer "B.Cu") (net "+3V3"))
 (segment (start 175.38 94) (end 175.38 93) (width 0.2) (layer "B.Cu") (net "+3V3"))
 (segment (start 172.60147 103.15) (end 170.875735 104.875735) (width 0.2) (layer "B.Cu") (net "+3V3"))
 (segment (start 162 89) (end 172 89) (width 0.2) (layer "B.Cu") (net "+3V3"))
 (segment (start 181 108) (end 179.9 109.1) (width 0.2) (layer "B.Cu") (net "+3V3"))
 (segment (start 175.5 103.15) (end 172.60147 103.15) (width 0.2) (layer "B.Cu") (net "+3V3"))
 (segment (start 146.135 93.39) (end 148.99 93.39) (width 0.2) (layer "F.Cu") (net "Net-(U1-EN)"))
 (segment (start 136.225 103.961522) (end 136.225 105.038478) (width 0.2) (layer "F.Cu") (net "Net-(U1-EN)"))
 (segment (start 144.025 95.5) (end 146.135 93.39) (width 0.2) (layer "F.Cu") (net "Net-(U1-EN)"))
 (segment (start 150.225 106.375) (end 147.05 103.2) (width 0.2) (layer "F.Cu") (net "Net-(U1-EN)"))
 (segment (start 168.275 108.325) (end 175.5 101.1) (width 0.2) (layer "F.Cu") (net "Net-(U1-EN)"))
 (segment (start 137.525 95.5) (end 144.025 95.5) (width 0.2) (layer "F.Cu") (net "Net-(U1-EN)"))
 (segment (start 151.275 92.055) (end 150.745 92.055) (width 0.2) (layer "F.Cu") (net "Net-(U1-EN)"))
 (segment (start 147.05 103.2) (end 136.986522 103.2) (width 0.2) (layer "F.Cu") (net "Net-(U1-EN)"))
 (segment (start 139.511522 108.325) (end 168.275 108.325) (width 0.2) (layer "F.Cu") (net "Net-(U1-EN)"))
 (segment (start 150.225 92.575) (end 150.225 106.375) (width 0.2) (layer "F.Cu") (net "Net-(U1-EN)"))
 (segment (start 136.225 105.038478) (end 139.511522 108.325) (width 0.2) (layer "F.Cu") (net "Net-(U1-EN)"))
 (segment (start 175.5 101.1) (end 175.5 100) (width 0.2) (layer "F.Cu") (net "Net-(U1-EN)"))
 (segment (start 148.99 93.39) (end 150.325 92.055) (width 0.2) (layer "F.Cu") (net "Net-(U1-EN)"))
 (segment (start 136.986522 103.2) (end 136.225 103.961522) (width 0.2) (layer "F.Cu") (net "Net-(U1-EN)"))
 (segment (start 150.325 92.055) (end 151.275 92.055) (width 0.2) (layer "F.Cu") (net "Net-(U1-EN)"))
 (segment (start 150.745 92.055) (end 150.225 92.575) (width 0.2) (layer "F.Cu") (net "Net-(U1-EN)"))
 (segment (start 182.585786 95) (end 183.414214 95) (width 0.2) (layer "B.Cu") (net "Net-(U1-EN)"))
 (segment (start 183.414214 95) (end 184 94.414214) (width 0.2) (layer "B.Cu") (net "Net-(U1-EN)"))
 (segment (start 176.6 98.9) (end 178.685786 98.9) (width 0.2) (layer "B.Cu") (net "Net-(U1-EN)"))
 (segment (start 184 94.414214) (end 184 92) (width 0.2) (layer "B.Cu") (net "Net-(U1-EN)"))
 (segment (start 184 92) (end 183 91) (width 0.2) (layer "B.Cu") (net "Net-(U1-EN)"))
 (segment (start 178.685786 98.9) (end 182.585786 95) (width 0.2) (layer "B.Cu") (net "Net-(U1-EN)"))
 (segment (start 175.5 100) (end 176.6 98.9) (width 0.2) (layer "B.Cu") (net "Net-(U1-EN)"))
 (segment (start 136.986522 96.8) (end 136.225 96.038478) (width 0.2) (layer "F.Cu") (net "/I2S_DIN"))
 (segment (start 144.71 92.99) (end 148.935 88.765) (width 0.2) (layer "F.Cu") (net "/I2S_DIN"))
 (segment (start 164.535 88.765) (end 167.825 92.055) (width 0.2) (layer "F.Cu") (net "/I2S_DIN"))
 (segment (start 148.935 88.765) (end 164.535 88.765) (width 0.2) (layer "F.Cu") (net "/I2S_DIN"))
 (segment (start 167.825 92.055) (end 168.775 92.055) (width 0.2) (layer "F.Cu") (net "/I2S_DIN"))
 (segment (start 148 101.246346) (end 143.553654 96.8) (width 0.2) (layer "F.Cu") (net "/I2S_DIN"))
 (segment (start 138.196522 92.99) (end 144.71 92.99) (width 0.2) (layer "F.Cu") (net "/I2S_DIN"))
 (segment (start 136.225 94.961522) (end 138.196522 92.99) (width 0.2) (layer "F.Cu") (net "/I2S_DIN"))
 (segment (start 143.553654 96.8) (end 136.986522 96.8) (width 0.2) (layer "F.Cu") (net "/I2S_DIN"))
 (segment (start 136.225 96.038478) (end 136.225 94.961522) (width 0.2) (layer "F.Cu") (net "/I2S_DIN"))
 (segment (start 148 102.16) (end 148 101.246346) (width 0.2) (layer "F.Cu") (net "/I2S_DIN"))
 (segment (start 154 102) (end 153.785 102.215) (width 0.2) (layer "F.Cu") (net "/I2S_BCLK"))
 (segment (start 153.785 102.215) (end 151.275 102.215) (width 0.2) (layer "F.Cu") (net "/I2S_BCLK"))
 (segment (start 146.38 98) (end 146 98) (width 0.2) (layer "F.Cu") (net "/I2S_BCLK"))
 (segment (start 148 99.62) (end 146.38 98) (width 0.2) (layer "F.Cu") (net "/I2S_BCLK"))
 (via (at 154 102) (size 0.6) (drill 0.3) (layers "F.Cu" "B.Cu") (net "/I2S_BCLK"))
 (via (at 146 98) (size 0.6) (drill 0.3) (layers "F.Cu" "B.Cu") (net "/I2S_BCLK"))
 (segment (start 146 98) (end 151 103) (width 0.2) (layer "B.Cu") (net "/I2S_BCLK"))
 (segment (start 153 103) (end 154 102) (width 0.2) (layer "B.Cu") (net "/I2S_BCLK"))
 (segment (start 151 103) (end 153 103) (width 0.2) (layer "B.Cu") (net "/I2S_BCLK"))
 (segment (start 153.055 100.945) (end 151.275 100.945) (width 0.2) (layer "F.Cu") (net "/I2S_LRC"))
 (segment (start 154 100) (end 153.055 100.945) (width 0.2) (layer "F.Cu") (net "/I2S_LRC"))
 (segment (start 148.08 97.08) (end 149 98) (width 0.2) (layer "F.Cu") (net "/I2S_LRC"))
 (segment (start 148 97.08) (end 148.08 97.08) (width 0.2) (layer "F.Cu") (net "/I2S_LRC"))
 (via (at 149 98) (size 0.6) (drill 0.3) (layers "F.Cu" "B.Cu") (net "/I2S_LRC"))
 (via (at 154 100) (size 0.6) (drill 0.3) (layers "F.Cu" "B.Cu") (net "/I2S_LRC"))
 (segment (start 149 98) (end 152 98) (width 0.2) (layer "B.Cu") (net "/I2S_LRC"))
 (segment (start 152 98) (end 154 100) (width 0.2) (layer "B.Cu") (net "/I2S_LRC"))
 (segment (start 168.775 93.325) (end 167.825 93.325) (width 0.2) (layer "F.Cu") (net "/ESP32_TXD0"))
 (segment (start 167.825 93.325) (end 167 94.15) (width 0.2) (layer "F.Cu") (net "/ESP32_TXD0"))
 (segment (start 172 97.761259) (end 172 97.08) (width 0.2) (layer "F.Cu") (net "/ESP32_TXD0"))
 (segment (start 167 94.15) (end 167 102) (width 0.2) (layer "F.Cu") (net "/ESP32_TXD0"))
 (segment (start 173.147371 98.90863) (end 172 97.761259) (width 0.2) (layer "F.Cu") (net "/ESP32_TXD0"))
 (via (at 173.147371 98.90863) (size 0.6) (drill 0.3) (layers "F.Cu" "B.Cu") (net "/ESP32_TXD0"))
 (via (at 167 102) (size 0.6) (drill 0.3) (layers "F.Cu" "B.Cu") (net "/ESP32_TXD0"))
 (segment (start 170.53 98.47) (end 172.708741 98.47) (width 0.2) (layer "B.Cu") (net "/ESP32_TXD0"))
 (segment (start 167 102) (end 170.53 98.47) (width 0.2) (layer "B.Cu") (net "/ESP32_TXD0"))
 (segment (start 172.708741 98.47) (end 173.147371 98.90863) (width 0.2) (layer "B.Cu") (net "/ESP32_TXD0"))
 (segment (start 171 96) (end 171 95.54) (width 0.2) (layer "F.Cu") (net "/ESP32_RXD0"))
 (segment (start 171 95.54) (end 172 94.54) (width 0.2) (layer "F.Cu") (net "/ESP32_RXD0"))
 (segment (start 168.775 94.595) (end 168.315837 94.595) (width 0.2) (layer "F.Cu") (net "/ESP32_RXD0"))
 (segment (start 168.315837 94.595) (end 167.994934 94.915903) (width 0.2) (layer "F.Cu") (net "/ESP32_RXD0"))
 (via (at 171 96) (size 0.6) (drill 0.3) (layers "F.Cu" "B.Cu") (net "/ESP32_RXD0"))
 (via (at 167.994934 94.915903) (size 0.6) (drill 0.3) (layers "F.Cu" "B.Cu") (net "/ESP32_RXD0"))
 (segment (start 167.994934 94.915903) (end 169.079031 96) (width 0.2) (layer "B.Cu") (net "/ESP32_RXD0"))
 (segment (start 169.079031 96) (end 171 96) (width 0.2) (layer "B.Cu") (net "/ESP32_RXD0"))
 (segment (start 137.525 91) (end 144.025 91) (width 0.2) (layer "F.Cu") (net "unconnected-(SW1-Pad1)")))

